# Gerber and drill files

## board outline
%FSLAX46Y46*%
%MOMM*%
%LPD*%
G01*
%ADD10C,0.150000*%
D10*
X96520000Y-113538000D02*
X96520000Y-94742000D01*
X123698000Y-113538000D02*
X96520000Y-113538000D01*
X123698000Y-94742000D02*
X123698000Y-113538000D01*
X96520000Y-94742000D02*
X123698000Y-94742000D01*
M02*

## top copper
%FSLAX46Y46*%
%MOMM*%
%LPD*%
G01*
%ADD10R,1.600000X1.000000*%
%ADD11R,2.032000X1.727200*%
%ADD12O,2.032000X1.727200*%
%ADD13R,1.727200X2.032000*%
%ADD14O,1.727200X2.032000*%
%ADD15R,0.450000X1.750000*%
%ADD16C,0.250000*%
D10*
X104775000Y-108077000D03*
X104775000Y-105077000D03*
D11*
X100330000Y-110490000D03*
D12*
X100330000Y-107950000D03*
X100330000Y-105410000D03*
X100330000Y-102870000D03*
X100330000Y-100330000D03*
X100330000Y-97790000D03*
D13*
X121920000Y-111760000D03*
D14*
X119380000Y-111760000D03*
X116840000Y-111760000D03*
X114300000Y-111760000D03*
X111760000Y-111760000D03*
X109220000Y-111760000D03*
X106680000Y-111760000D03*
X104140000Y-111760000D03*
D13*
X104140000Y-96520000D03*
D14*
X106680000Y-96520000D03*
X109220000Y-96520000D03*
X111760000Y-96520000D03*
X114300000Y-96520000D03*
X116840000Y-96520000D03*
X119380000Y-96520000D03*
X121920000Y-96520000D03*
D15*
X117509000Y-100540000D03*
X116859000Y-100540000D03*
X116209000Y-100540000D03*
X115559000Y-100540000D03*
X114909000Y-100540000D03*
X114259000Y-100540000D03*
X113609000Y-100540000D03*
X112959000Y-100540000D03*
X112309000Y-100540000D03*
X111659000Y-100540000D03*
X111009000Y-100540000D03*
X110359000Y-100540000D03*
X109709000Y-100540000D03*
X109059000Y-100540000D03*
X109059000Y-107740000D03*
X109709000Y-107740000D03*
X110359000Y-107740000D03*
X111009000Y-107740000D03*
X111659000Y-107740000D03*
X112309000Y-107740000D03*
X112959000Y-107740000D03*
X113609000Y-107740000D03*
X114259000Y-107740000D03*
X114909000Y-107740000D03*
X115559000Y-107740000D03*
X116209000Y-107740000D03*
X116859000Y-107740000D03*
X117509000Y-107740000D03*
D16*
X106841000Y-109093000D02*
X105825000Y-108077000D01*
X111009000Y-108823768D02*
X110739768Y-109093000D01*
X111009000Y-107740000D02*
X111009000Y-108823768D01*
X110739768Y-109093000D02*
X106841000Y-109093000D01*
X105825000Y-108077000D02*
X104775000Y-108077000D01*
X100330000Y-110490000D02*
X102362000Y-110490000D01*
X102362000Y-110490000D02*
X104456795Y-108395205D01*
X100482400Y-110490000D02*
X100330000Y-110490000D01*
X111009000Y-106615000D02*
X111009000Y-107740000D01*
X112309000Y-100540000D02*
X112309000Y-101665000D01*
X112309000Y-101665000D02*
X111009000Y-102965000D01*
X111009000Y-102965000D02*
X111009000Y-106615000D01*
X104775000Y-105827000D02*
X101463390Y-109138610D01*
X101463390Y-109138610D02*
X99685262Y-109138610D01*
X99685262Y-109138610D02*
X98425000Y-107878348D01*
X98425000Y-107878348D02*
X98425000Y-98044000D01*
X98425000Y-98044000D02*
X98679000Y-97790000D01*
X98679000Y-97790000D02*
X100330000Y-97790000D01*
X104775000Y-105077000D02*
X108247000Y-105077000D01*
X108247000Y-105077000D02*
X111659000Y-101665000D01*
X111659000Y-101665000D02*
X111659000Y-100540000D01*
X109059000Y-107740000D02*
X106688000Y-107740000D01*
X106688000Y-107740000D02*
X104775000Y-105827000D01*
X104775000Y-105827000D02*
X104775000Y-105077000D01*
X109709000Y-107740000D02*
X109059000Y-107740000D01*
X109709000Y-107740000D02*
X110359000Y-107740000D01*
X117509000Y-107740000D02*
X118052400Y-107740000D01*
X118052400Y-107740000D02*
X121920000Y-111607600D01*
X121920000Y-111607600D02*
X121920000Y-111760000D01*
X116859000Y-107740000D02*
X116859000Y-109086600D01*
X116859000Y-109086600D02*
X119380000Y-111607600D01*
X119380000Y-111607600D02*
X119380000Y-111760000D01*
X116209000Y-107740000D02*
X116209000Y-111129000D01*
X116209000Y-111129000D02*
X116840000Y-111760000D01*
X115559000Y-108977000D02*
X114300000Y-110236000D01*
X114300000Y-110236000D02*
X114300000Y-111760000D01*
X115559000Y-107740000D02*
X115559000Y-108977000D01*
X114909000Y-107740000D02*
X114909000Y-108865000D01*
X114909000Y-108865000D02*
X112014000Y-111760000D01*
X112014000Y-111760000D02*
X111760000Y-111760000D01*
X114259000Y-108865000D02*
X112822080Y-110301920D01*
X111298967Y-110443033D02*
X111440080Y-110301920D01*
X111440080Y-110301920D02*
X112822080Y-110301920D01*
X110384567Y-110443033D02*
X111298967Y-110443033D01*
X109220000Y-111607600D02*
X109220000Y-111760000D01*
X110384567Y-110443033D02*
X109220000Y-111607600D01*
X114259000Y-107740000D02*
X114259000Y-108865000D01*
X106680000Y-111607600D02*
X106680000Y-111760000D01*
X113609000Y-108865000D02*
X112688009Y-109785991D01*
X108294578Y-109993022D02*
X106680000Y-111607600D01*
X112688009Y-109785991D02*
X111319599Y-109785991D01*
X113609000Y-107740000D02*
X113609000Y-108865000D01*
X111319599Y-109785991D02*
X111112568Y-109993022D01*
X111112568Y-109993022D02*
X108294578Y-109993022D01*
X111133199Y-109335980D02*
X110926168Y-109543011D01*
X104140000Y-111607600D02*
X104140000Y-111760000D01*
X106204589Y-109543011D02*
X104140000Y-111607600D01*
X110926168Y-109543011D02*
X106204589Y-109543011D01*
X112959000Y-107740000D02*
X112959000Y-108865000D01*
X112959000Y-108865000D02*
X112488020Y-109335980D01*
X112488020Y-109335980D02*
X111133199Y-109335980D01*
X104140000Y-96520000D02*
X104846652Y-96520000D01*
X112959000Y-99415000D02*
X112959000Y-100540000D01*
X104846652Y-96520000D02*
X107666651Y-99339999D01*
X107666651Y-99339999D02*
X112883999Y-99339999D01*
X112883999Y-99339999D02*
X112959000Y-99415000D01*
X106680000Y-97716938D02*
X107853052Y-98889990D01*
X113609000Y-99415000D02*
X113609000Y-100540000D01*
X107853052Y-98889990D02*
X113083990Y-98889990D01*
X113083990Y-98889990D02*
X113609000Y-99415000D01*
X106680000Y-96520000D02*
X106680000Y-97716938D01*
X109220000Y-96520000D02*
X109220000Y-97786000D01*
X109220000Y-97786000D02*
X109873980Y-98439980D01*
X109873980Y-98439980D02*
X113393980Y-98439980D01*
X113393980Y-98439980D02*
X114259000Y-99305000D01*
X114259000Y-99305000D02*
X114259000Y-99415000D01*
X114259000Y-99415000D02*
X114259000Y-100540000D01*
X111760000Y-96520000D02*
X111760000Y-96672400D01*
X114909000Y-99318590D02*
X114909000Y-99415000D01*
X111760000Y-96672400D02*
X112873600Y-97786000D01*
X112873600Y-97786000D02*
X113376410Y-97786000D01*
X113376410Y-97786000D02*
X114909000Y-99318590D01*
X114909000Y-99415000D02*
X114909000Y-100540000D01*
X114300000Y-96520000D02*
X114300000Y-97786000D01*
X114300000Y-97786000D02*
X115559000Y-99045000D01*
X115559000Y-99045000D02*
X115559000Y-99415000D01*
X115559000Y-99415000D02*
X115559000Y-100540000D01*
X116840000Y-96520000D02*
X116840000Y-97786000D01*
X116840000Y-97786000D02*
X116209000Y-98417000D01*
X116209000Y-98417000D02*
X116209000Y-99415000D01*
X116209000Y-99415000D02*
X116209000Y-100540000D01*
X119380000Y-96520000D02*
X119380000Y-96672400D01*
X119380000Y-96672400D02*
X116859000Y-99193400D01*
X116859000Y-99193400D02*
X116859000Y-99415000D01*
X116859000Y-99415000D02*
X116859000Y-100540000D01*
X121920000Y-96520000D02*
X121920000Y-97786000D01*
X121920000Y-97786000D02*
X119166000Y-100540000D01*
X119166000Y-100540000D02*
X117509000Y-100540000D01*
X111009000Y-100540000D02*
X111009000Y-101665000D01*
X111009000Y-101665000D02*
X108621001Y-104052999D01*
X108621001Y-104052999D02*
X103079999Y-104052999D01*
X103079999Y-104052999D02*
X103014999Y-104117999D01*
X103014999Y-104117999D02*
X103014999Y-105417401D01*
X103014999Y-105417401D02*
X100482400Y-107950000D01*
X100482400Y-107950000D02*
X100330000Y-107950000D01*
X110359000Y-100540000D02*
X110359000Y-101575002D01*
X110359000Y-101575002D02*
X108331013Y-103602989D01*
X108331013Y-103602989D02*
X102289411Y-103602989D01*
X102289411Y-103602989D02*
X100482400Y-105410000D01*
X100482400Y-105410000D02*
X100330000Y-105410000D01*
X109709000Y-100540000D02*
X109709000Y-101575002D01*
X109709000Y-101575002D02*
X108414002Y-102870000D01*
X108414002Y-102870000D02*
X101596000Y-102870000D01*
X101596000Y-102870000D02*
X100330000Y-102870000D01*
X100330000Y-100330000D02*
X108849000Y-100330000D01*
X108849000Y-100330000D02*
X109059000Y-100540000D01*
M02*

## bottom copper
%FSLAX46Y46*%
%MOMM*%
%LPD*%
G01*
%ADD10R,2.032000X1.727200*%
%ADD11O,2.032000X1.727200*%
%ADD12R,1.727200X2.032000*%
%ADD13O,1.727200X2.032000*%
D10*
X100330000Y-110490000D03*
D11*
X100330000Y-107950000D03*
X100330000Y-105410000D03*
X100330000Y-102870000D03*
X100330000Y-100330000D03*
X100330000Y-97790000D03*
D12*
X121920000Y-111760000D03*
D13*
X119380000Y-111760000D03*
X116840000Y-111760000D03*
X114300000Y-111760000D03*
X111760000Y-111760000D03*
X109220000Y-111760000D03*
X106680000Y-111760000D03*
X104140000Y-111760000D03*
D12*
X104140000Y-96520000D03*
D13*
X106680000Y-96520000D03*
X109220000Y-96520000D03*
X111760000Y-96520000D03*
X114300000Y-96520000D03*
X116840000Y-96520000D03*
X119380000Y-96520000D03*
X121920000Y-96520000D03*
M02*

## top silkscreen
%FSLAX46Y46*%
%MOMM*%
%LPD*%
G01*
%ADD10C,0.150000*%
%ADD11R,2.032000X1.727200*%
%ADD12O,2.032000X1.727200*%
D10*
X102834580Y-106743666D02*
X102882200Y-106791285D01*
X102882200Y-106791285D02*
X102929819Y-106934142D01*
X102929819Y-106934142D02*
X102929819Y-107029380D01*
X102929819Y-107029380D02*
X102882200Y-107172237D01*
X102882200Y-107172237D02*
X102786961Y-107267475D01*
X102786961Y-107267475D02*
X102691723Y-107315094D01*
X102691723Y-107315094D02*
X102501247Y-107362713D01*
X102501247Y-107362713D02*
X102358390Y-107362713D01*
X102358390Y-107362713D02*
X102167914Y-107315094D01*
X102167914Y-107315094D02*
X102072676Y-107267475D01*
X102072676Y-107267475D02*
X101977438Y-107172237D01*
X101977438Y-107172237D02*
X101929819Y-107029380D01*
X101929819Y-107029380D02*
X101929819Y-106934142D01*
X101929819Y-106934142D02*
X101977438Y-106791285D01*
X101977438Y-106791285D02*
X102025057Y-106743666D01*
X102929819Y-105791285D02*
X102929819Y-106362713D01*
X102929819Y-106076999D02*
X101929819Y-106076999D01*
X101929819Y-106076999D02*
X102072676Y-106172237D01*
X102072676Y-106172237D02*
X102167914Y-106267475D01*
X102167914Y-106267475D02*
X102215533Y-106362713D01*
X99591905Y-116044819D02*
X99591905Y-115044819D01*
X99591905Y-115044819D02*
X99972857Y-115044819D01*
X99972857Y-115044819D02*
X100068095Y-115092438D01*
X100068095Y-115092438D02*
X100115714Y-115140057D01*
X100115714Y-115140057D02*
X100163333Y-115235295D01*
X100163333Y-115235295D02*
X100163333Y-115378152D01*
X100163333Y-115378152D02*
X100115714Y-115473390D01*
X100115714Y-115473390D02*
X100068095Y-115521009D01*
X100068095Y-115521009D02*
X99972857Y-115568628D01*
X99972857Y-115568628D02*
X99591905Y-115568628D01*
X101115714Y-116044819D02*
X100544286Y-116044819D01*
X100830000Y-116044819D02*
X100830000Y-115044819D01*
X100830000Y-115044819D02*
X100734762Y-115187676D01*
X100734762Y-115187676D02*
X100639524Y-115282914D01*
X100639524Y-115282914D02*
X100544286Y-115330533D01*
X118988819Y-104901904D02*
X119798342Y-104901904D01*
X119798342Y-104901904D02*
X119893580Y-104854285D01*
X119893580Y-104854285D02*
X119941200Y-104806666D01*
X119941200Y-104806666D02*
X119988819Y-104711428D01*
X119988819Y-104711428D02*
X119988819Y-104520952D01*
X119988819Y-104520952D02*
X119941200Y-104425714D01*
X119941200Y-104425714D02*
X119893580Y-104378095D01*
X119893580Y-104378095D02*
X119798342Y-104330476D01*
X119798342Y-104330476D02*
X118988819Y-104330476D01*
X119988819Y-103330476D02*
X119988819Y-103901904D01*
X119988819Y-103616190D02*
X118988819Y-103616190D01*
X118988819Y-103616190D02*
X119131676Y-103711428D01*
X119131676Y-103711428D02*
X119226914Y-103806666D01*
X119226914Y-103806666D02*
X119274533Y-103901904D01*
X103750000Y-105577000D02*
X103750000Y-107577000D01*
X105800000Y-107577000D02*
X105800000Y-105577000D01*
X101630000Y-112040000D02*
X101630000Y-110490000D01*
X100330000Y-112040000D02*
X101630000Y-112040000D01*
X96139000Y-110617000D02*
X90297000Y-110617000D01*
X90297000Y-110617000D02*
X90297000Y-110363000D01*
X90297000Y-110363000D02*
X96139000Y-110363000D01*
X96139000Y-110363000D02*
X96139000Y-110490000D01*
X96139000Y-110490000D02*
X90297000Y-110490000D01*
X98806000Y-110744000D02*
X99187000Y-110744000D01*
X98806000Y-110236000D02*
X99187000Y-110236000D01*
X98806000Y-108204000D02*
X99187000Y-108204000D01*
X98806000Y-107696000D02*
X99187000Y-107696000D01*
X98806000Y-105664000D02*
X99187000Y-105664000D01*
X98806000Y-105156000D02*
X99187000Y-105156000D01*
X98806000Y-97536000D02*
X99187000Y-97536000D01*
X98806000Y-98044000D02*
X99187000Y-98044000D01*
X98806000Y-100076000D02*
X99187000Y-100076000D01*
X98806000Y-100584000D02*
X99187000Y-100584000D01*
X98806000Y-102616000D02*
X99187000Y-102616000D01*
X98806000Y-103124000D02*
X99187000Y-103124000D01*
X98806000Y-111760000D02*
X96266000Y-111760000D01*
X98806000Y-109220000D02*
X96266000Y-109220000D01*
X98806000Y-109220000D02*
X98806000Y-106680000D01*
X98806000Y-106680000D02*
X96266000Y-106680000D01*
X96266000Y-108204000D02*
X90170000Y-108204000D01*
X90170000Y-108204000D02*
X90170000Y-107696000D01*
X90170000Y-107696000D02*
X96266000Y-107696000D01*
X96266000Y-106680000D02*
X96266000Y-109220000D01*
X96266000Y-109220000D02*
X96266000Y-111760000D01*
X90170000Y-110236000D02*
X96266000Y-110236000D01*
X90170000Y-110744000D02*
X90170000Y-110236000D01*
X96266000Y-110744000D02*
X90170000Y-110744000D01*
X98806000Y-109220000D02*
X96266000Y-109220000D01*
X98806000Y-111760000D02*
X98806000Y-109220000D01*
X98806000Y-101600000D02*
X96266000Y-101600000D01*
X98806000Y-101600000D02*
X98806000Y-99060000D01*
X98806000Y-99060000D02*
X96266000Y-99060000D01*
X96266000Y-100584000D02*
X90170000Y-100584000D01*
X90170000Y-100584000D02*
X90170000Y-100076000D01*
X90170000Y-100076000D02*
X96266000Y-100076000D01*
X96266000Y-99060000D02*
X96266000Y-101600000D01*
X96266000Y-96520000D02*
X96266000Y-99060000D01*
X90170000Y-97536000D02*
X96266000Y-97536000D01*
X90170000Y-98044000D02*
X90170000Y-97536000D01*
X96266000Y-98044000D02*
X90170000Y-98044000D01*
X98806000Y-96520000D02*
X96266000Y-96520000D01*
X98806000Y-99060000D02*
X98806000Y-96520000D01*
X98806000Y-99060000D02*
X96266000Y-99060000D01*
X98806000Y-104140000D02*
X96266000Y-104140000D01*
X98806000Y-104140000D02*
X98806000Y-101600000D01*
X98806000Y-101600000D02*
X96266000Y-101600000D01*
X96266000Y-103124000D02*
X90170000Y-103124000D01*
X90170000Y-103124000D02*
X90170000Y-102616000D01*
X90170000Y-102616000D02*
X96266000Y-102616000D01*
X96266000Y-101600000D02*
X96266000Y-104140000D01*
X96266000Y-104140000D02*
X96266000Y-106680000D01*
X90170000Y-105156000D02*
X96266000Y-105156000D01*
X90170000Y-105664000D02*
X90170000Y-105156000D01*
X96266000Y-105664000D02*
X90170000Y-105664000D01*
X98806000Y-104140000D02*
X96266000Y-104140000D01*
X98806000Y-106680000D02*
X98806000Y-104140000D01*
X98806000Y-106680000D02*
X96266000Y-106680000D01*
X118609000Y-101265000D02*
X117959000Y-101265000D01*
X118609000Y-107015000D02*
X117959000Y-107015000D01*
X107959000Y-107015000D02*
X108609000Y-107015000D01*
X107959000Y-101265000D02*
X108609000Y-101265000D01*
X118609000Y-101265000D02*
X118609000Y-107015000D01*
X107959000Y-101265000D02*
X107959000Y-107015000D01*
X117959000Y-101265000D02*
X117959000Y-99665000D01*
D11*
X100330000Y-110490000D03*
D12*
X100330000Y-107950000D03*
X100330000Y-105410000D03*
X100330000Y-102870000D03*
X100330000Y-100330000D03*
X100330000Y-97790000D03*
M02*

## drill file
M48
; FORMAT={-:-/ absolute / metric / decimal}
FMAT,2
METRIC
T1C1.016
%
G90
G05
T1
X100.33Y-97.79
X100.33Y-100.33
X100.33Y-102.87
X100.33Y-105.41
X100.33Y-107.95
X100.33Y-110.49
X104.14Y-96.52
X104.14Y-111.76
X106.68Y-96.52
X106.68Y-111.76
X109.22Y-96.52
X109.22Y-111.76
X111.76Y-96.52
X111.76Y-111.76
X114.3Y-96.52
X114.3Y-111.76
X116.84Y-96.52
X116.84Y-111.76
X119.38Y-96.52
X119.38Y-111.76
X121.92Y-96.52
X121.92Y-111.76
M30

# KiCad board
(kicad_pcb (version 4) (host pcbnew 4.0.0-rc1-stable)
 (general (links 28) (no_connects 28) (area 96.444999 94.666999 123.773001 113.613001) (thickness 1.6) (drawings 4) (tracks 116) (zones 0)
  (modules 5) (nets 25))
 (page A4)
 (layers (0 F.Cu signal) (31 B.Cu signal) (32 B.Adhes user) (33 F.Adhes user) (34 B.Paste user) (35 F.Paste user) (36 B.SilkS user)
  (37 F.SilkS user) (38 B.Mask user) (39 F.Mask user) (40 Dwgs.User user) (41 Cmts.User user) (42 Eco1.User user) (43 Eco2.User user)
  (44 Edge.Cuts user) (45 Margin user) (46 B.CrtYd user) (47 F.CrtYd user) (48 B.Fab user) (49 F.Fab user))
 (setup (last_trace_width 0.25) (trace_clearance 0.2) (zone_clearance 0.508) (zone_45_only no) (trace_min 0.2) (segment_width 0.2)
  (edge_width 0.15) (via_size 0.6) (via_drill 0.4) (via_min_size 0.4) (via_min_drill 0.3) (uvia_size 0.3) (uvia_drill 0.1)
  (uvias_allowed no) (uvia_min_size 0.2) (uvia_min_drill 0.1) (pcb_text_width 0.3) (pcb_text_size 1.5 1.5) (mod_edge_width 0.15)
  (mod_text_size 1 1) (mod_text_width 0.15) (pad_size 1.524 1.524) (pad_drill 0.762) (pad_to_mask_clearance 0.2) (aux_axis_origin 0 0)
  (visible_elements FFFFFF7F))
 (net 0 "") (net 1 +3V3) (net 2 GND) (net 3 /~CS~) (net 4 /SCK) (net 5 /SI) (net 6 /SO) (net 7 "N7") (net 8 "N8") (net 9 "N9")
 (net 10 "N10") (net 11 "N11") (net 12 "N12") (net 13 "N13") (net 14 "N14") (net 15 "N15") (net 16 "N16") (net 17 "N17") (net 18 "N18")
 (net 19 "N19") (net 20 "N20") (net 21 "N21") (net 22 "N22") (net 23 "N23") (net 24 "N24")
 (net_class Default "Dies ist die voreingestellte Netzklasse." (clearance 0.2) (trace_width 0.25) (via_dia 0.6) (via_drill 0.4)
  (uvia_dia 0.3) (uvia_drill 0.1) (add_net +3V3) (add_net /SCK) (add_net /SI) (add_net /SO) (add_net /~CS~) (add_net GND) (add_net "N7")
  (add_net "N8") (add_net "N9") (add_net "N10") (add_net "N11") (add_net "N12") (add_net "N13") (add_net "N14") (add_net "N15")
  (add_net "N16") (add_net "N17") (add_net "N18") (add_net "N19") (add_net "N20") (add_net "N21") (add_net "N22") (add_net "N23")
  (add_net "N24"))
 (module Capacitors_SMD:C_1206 (layer F.Cu) (at 104.775 106.577 90)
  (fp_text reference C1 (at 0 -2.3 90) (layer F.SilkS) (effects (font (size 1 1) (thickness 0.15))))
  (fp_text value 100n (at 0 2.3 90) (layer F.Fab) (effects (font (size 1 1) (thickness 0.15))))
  (fp_line (start 1 -1.025) (end -1 -1.025) (layer F.SilkS) (width 0.15))
  (fp_line (start -1 1.025) (end 1 1.025) (layer F.SilkS) (width 0.15))
  (pad 1 smd rect (at -1.5 0 90) (size 1 1.6) (layers F.Cu F.Paste F.Mask) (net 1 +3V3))
  (pad 2 smd rect (at 1.5 0 90) (size 1 1.6) (layers F.Cu F.Paste F.Mask) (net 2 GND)))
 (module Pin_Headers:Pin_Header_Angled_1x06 (layer F.Cu) (at 100.33 110.49 180)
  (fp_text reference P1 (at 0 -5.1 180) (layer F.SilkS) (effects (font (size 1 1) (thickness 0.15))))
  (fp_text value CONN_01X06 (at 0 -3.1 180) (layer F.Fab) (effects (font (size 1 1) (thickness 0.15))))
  (fp_line (start -1.3 -1.55) (end -1.3 0) (layer F.SilkS) (width 0.15))
  (fp_line (start 0 -1.55) (end -1.3 -1.55) (layer F.SilkS) (width 0.15))
  (fp_line (start 4.191 -0.127) (end 10.033 -0.127) (layer F.SilkS) (width 0.15))
  (fp_line (start 10.033 -0.127) (end 10.033 0.127) (layer F.SilkS) (width 0.15))
  (fp_line (start 10.033 0.127) (end 4.191 0.127) (layer F.SilkS) (width 0.15))
  (fp_line (start 4.191 0.127) (end 4.191 0) (layer F.SilkS) (width 0.15))
  (fp_line (start 4.191 0) (end 10.033 0) (layer F.SilkS) (width 0.15))
  (fp_line (start 1.524 -0.254) (end 1.143 -0.254) (layer F.SilkS) (width 0.15))
  (fp_line (start 1.524 0.254) (end 1.143 0.254) (layer F.SilkS) (width 0.15))
  (fp_line (start 1.524 2.286) (end 1.143 2.286) (layer F.SilkS) (width 0.15))
  (fp_line (start 1.524 2.794) (end 1.143 2.794) (layer F.SilkS) (width 0.15))
  (fp_line (start 1.524 4.826) (end 1.143 4.826) (layer F.SilkS) (width 0.15))
  (fp_line (start 1.524 5.334) (end 1.143 5.334) (layer F.SilkS) (width 0.15))
  (fp_line (start 1.524 12.954) (end 1.143 12.954) (layer F.SilkS) (width 0.15))
  (fp_line (start 1.524 12.446) (end 1.143 12.446) (layer F.SilkS) (width 0.15))
  (fp_line (start 1.524 10.414) (end 1.143 10.414) (layer F.SilkS) (width 0.15))
  (fp_line (start 1.524 9.906) (end 1.143 9.906) (layer F.SilkS) (width 0.15))
  (fp_line (start 1.524 7.874) (end 1.143 7.874) (layer F.SilkS) (width 0.15))
  (fp_line (start 1.524 7.366) (end 1.143 7.366) (layer F.SilkS) (width 0.15))
  (fp_line (start 1.524 -1.27) (end 4.064 -1.27) (layer F.SilkS) (width 0.15))
  (fp_line (start 1.524 1.27) (end 4.064 1.27) (layer F.SilkS) (width 0.15))
  (fp_line (start 1.524 1.27) (end 1.524 3.81) (layer F.SilkS) (width 0.15))
  (fp_line (start 1.524 3.81) (end 4.064 3.81) (layer F.SilkS) (width 0.15))
  (fp_line (start 4.064 2.286) (end 10.16 2.286) (layer F.SilkS) (width 0.15))
  (fp_line (start 10.16 2.286) (end 10.16 2.794) (layer F.SilkS) (width 0.15))
  (fp_line (start 10.16 2.794) (end 4.064 2.794) (layer F.SilkS) (width 0.15))
  (fp_line (start 4.064 3.81) (end 4.064 1.27) (layer F.SilkS) (width 0.15))
  (fp_line (start 4.064 1.27) (end 4.064 -1.27) (layer F.SilkS) (width 0.15))
  (fp_line (start 10.16 0.254) (end 4.064 0.254) (layer F.SilkS) (width 0.15))
  (fp_line (start 10.16 -0.254) (end 10.16 0.254) (layer F.SilkS) (width 0.15))
  (fp_line (start 4.064 -0.254) (end 10.16 -0.254) (layer F.SilkS) (width 0.15))
  (fp_line (start 1.524 1.27) (end 4.064 1.27) (layer F.SilkS) (width 0.15))
  (fp_line (start 1.524 -1.27) (end 1.524 1.27) (layer F.SilkS) (width 0.15))
  (fp_line (start 1.524 8.89) (end 4.064 8.89) (layer F.SilkS) (width 0.15))
  (fp_line (start 1.524 8.89) (end 1.524 11.43) (layer F.SilkS) (width 0.15))
  (fp_line (start 1.524 11.43) (end 4.064 11.43) (layer F.SilkS) (width 0.15))
  (fp_line (start 4.064 9.906) (end 10.16 9.906) (layer F.SilkS) (width 0.15))
  (fp_line (start 10.16 9.906) (end 10.16 10.414) (layer F.SilkS) (width 0.15))
  (fp_line (start 10.16 10.414) (end 4.064 10.414) (layer F.SilkS) (width 0.15))
  (fp_line (start 4.064 11.43) (end 4.064 8.89) (layer F.SilkS) (width 0.15))
  (fp_line (start 4.064 13.97) (end 4.064 11.43) (layer F.SilkS) (width 0.15))
  (fp_line (start 10.16 12.954) (end 4.064 12.954) (layer F.SilkS) (width 0.15))
  (fp_line (start 10.16 12.446) (end 10.16 12.954) (layer F.SilkS) (width 0.15))
  (fp_line (start 4.064 12.446) (end 10.16 12.446) (layer F.SilkS) (width 0.15))
  (fp_line (start 1.524 13.97) (end 4.064 13.97) (layer F.SilkS) (width 0.15))
  (fp_line (start 1.524 11.43) (end 1.524 13.97) (layer F.SilkS) (width 0.15))
  (fp_line (start 1.524 11.43) (end 4.064 11.43) (layer F.SilkS) (width 0.15))
  (fp_line (start 1.524 6.35) (end 4.064 6.35) (layer F.SilkS) (width 0.15))
  (fp_line (start 1.524 6.35) (end 1.524 8.89) (layer F.SilkS) (width 0.15))
  (fp_line (start 1.524 8.89) (end 4.064 8.89) (layer F.SilkS) (width 0.15))
  (fp_line (start 4.064 7.366) (end 10.16 7.366) (layer F.SilkS) (width 0.15))
  (fp_line (start 10.16 7.366) (end 10.16 7.874) (layer F.SilkS) (width 0.15))
  (fp_line (start 10.16 7.874) (end 4.064 7.874) (layer F.SilkS) (width 0.15))
  (fp_line (start 4.064 8.89) (end 4.064 6.35) (layer F.SilkS) (width 0.15))
  (fp_line (start 4.064 6.35) (end 4.064 3.81) (layer F.SilkS) (width 0.15))
  (fp_line (start 10.16 5.334) (end 4.064 5.334) (layer F.SilkS) (width 0.15))
  (fp_line (start 10.16 4.826) (end 10.16 5.334) (layer F.SilkS) (width 0.15))
  (fp_line (start 4.064 4.826) (end 10.16 4.826) (layer F.SilkS) (width 0.15))
  (fp_line (start 1.524 6.35) (end 4.064 6.35) (layer F.SilkS) (width 0.15))
  (fp_line (start 1.524 3.81) (end 1.524 6.35) (layer F.SilkS) (width 0.15))
  (fp_line (start 1.524 3.81) (end 4.064 3.81) (layer F.SilkS) (width 0.15))
  (pad 1 thru_hole rect (at 0 0 180) (size 2.032 1.7272) (drill 1.016) (layers *.Cu *.Mask F.SilkS) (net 1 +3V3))
  (pad 2 thru_hole oval (at 0 2.54 180) (size 2.032 1.7272) (drill 1.016) (layers *.Cu *.Mask F.SilkS) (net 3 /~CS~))
  (pad 3 thru_hole oval (at 0 5.08 180) (size 2.032 1.7272) (drill 1.016) (layers *.Cu *.Mask F.SilkS) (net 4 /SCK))
  (pad 4 thru_hole oval (at 0 7.62 180) (size 2.032 1.7272) (drill 1.016) (layers *.Cu *.Mask F.SilkS) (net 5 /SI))
  (pad 5 thru_hole oval (at 0 10.16 180) (size 2.032 1.7272) (drill 1.016) (layers *.Cu *.Mask F.SilkS) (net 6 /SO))
  (pad 6 thru_hole oval (at 0 12.7 180) (size 2.032 1.7272) (drill 1.016) (layers *.Cu *.Mask F.SilkS) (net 2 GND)))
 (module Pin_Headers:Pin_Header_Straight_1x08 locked (layer B.Cu) (at 121.92 111.76 90)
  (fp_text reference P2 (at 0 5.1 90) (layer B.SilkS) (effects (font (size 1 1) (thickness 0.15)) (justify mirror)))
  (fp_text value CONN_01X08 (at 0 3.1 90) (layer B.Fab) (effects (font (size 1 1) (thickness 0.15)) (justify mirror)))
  (pad 1 thru_hole rect (at 0 0 90) (size 2.032 1.7272) (drill 1.016) (layers *.Cu *.Mask B.SilkS) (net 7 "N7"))
  (pad 2 thru_hole oval (at 0 -2.54 90) (size 2.032 1.7272) (drill 1.016) (layers *.Cu *.Mask B.SilkS) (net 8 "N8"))
  (pad 3 thru_hole oval (at 0 -5.08 90) (size 2.032 1.7272) (drill 1.016) (layers *.Cu *.Mask B.SilkS) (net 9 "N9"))
  (pad 4 thru_hole oval (at 0 -7.62 90) (size 2.032 1.7272) (drill 1.016) (layers *.Cu *.Mask B.SilkS) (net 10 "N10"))
  (pad 5 thru_hole oval (at 0 -10.16 90) (size 2.032 1.7272) (drill 1.016) (layers *.Cu *.Mask B.SilkS) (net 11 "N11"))
  (pad 6 thru_hole oval (at 0 -12.7 90) (size 2.032 1.7272) (drill 1.016) (layers *.Cu *.Mask B.SilkS) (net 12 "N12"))
  (pad 7 thru_hole oval (at 0 -15.24 90) (size 2.032 1.7272) (drill 1.016) (layers *.Cu *.Mask B.SilkS) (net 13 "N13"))
  (pad 8 thru_hole oval (at 0 -17.78 90) (size 2.032 1.7272) (drill 1.016) (layers *.Cu *.Mask B.SilkS) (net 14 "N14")))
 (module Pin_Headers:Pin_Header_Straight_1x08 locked (layer B.Cu) (at 104.14 96.52 270)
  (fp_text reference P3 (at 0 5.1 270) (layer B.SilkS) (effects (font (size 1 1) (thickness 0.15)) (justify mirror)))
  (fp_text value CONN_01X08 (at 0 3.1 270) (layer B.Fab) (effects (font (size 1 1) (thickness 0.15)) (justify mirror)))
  (pad 1 thru_hole rect (at 0 0 270) (size 2.032 1.7272) (drill 1.016) (layers *.Cu *.Mask B.SilkS) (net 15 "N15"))
  (pad 2 thru_hole oval (at 0 -2.54 270) (size 2.032 1.7272) (drill 1.016) (layers *.Cu *.Mask B.SilkS) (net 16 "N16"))
  (pad 3 thru_hole oval (at 0 -5.08 270) (size 2.032 1.7272) (drill 1.016) (layers *.Cu *.Mask B.SilkS) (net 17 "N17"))
  (pad 4 thru_hole oval (at 0 -7.62 270) (size 2.032 1.7272) (drill 1.016) (layers *.Cu *.Mask B.SilkS) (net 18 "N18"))
  (pad 5 thru_hole oval (at 0 -10.16 270) (size 2.032 1.7272) (drill 1.016) (layers *.Cu *.Mask B.SilkS) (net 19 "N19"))
  (pad 6 thru_hole oval (at 0 -12.7 270) (size 2.032 1.7272) (drill 1.016) (layers *.Cu *.Mask B.SilkS) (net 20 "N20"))
  (pad 7 thru_hole oval (at 0 -15.24 270) (size 2.032 1.7272) (drill 1.016) (layers *.Cu *.Mask B.SilkS) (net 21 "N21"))
  (pad 8 thru_hole oval (at 0 -17.78 270) (size 2.032 1.7272) (drill 1.016) (layers *.Cu *.Mask B.SilkS) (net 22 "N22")))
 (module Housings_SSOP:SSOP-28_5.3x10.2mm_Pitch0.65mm (layer F.Cu) (at 113.284 104.14 270)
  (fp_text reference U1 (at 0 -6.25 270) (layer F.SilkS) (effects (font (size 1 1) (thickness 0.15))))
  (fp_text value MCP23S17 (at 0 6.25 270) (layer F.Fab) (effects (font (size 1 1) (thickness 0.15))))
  (fp_line (start -2.875 -5.325) (end -2.875 -4.675) (layer F.SilkS) (width 0.15))
  (fp_line (start 2.875 -5.325) (end 2.875 -4.675) (layer F.SilkS) (width 0.15))
  (fp_line (start 2.875 5.325) (end 2.875 4.675) (layer F.SilkS) (width 0.15))
  (fp_line (start -2.875 5.325) (end -2.875 4.675) (layer F.SilkS) (width 0.15))
  (fp_line (start -2.875 -5.325) (end 2.875 -5.325) (layer F.SilkS) (width 0.15))
  (fp_line (start -2.875 5.325) (end 2.875 5.325) (layer F.SilkS) (width 0.15))
  (fp_line (start -2.875 -4.675) (end -4.475 -4.675) (layer F.SilkS) (width 0.15))
  (pad 1 smd rect (at -3.6 -4.225 270) (size 1.75 0.45) (layers F.Cu F.Paste F.Mask) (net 22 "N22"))
  (pad 2 smd rect (at -3.6 -3.575 270) (size 1.75 0.45) (layers F.Cu F.Paste F.Mask) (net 21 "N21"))
  (pad 3 smd rect (at -3.6 -2.925 270) (size 1.75 0.45) (layers F.Cu F.Paste F.Mask) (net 20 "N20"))
  (pad 4 smd rect (at -3.6 -2.275 270) (size 1.75 0.45) (layers F.Cu F.Paste F.Mask) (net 19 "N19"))
  (pad 5 smd rect (at -3.6 -1.625 270) (size 1.75 0.45) (layers F.Cu F.Paste F.Mask) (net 18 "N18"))
  (pad 6 smd rect (at -3.6 -0.975 270) (size 1.75 0.45) (layers F.Cu F.Paste F.Mask) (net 17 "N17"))
  (pad 7 smd rect (at -3.6 -0.325 270) (size 1.75 0.45) (layers F.Cu F.Paste F.Mask) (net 16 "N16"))
  (pad 8 smd rect (at -3.6 0.325 270) (size 1.75 0.45) (layers F.Cu F.Paste F.Mask) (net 15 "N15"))
  (pad 9 smd rect (at -3.6 0.975 270) (size 1.75 0.45) (layers F.Cu F.Paste F.Mask) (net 1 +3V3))
  (pad 10 smd rect (at -3.6 1.625 270) (size 1.75 0.45) (layers F.Cu F.Paste F.Mask) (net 2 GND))
  (pad 11 smd rect (at -3.6 2.275 270) (size 1.75 0.45) (layers F.Cu F.Paste F.Mask) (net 3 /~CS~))
  (pad 12 smd rect (at -3.6 2.925 270) (size 1.75 0.45) (layers F.Cu F.Paste F.Mask) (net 4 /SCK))
  (pad 13 smd rect (at -3.6 3.575 270) (size 1.75 0.45) (layers F.Cu F.Paste F.Mask) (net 5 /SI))
  (pad 14 smd rect (at -3.6 4.225 270) (size 1.75 0.45) (layers F.Cu F.Paste F.Mask) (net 6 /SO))
  (pad 15 smd rect (at 3.6 4.225 270) (size 1.75 0.45) (layers F.Cu F.Paste F.Mask) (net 2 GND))
  (pad 16 smd rect (at 3.6 3.575 270) (size 1.75 0.45) (layers F.Cu F.Paste F.Mask) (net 2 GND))
  (pad 17 smd rect (at 3.6 2.925 270) (size 1.75 0.45) (layers F.Cu F.Paste F.Mask) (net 2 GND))
  (pad 18 smd rect (at 3.6 2.275 270) (size 1.75 0.45) (layers F.Cu F.Paste F.Mask) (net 1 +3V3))
  (pad 19 smd rect (at 3.6 1.625 270) (size 1.75 0.45) (layers F.Cu F.Paste F.Mask) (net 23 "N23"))
  (pad 20 smd rect (at 3.6 0.975 270) (size 1.75 0.45) (layers F.Cu F.Paste F.Mask) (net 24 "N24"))
  (pad 21 smd rect (at 3.6 0.325 270) (size 1.75 0.45) (layers F.Cu F.Paste F.Mask) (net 14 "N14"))
  (pad 22 smd rect (at 3.6 -0.325 270) (size 1.75 0.45) (layers F.Cu F.Paste F.Mask) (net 13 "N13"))
  (pad 23 smd rect (at 3.6 -0.975 270) (size 1.75 0.45) (layers F.Cu F.Paste F.Mask) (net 12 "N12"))
  (pad 24 smd rect (at 3.6 -1.625 270) (size 1.75 0.45) (layers F.Cu F.Paste F.Mask) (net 11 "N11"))
  (pad 25 smd rect (at 3.6 -2.275 270) (size 1.75 0.45) (layers F.Cu F.Paste F.Mask) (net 10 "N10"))
  (pad 26 smd rect (at 3.6 -2.925 270) (size 1.75 0.45) (layers F.Cu F.Paste F.Mask) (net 9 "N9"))
  (pad 27 smd rect (at 3.6 -3.575 270) (size 1.75 0.45) (layers F.Cu F.Paste F.Mask) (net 8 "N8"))
  (pad 28 smd rect (at 3.6 -4.225 270) (size 1.75 0.45) (layers F.Cu F.Paste F.Mask) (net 7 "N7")))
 (gr_line (start 96.52 113.538) (end 96.52 94.742) (layer Edge.Cuts) (width 0.15))
 (gr_line (start 123.698 113.538) (end 96.52 113.538) (layer Edge.Cuts) (width 0.15))
 (gr_line (start 123.698 94.742) (end 123.698 113.538) (layer Edge.Cuts) (width 0.15))
 (gr_line (start 96.52 94.742) (end 123.698 94.742) (layer Edge.Cuts) (width 0.15))
 (segment (start 106.841 109.093) (end 105.825 108.077) (width 0.25) (layer F.Cu) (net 1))
 (segment (start 111.009 108.823768) (end 110.739768 109.093) (width 0.25) (layer F.Cu) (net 1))
 (segment (start 111.009 107.74) (end 111.009 108.823768) (width 0.25) (layer F.Cu) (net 1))
 (segment (start 110.739768 109.093) (end 106.841 109.093) (width 0.25) (layer F.Cu) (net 1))
 (segment (start 105.825 108.077) (end 104.775 108.077) (width 0.25) (layer F.Cu) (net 1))
 (segment (start 100.33 110.49) (end 102.362 110.49) (width 0.25) (layer F.Cu) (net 1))
 (segment (start 102.362 110.49) (end 104.456795 108.395205) (width 0.25) (layer F.Cu) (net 1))
 (segment (start 100.4824 110.49) (end 100.33 110.49) (width 0.25) (layer F.Cu) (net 1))
 (segment (start 111.009 106.615) (end 111.009 107.74) (width 0.25) (layer F.Cu) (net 1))
 (segment (start 112.309 100.54) (end 112.309 101.665) (width 0.25) (layer F.Cu) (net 1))
 (segment (start 112.309 101.665) (end 111.009 102.965) (width 0.25) (layer F.Cu) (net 1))
 (segment (start 111.009 102.965) (end 111.009 106.615) (width 0.25) (layer F.Cu) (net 1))
 (segment (start 104.775 105.827) (end 101.46339 109.13861) (width 0.25) (layer F.Cu) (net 2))
 (segment (start 101.46339 109.13861) (end 99.685262 109.13861) (width 0.25) (layer F.Cu) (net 2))
 (segment (start 99.685262 109.13861) (end 98.425 107.878348) (width 0.25) (layer F.Cu) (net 2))
 (segment (start 98.425 107.878348) (end 98.425 98.044) (width 0.25) (layer F.Cu) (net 2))
 (segment (start 98.425 98.044) (end 98.679 97.79) (width 0.25) (layer F.Cu) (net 2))
 (segment (start 98.679 97.79) (end 100.33 97.79) (width 0.25) (layer F.Cu) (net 2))
 (segment (start 104.775 105.077) (end 108.247 105.077) (width 0.25) (layer F.Cu) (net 2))
 (segment (start 108.247 105.077) (end 111.659 101.665) (width 0.25) (layer F.Cu) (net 2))
 (segment (start 111.659 101.665) (end 111.659 100.54) (width 0.25) (layer F.Cu) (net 2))
 (segment (start 109.059 107.74) (end 106.688 107.74) (width 0.25) (layer F.Cu) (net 2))
 (segment (start 106.688 107.74) (end 104.775 105.827) (width 0.25) (layer F.Cu) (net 2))
 (segment (start 104.775 105.827) (end 104.775 105.077) (width 0.25) (layer F.Cu) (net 2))
 (segment (start 109.709 107.74) (end 109.059 107.74) (width 0.25) (layer F.Cu) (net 2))
 (segment (start 109.709 107.74) (end 110.359 107.74) (width 0.25) (layer F.Cu) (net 2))
 (segment (start 117.509 107.74) (end 118.0524 107.74) (width 0.25) (layer F.Cu) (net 7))
 (segment (start 118.0524 107.74) (end 121.92 111.6076) (width 0.25) (layer F.Cu) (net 7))
 (segment (start 121.92 111.6076) (end 121.92 111.76) (width 0.25) (layer F.Cu) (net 7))
 (segment (start 116.859 107.74) (end 116.859 109.0866) (width 0.25) (layer F.Cu) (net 8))
 (segment (start 116.859 109.0866) (end 119.38 111.6076) (width 0.25) (layer F.Cu) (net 8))
 (segment (start 119.38 111.6076) (end 119.38 111.76) (width 0.25) (layer F.Cu) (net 8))
 (segment (start 116.209 107.74) (end 116.209 111.129) (width 0.25) (layer F.Cu) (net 9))
 (segment (start 116.209 111.129) (end 116.84 111.76) (width 0.25) (layer F.Cu) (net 9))
 (segment (start 115.559 108.977) (end 114.3 110.236) (width 0.25) (layer F.Cu) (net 10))
 (segment (start 114.3 110.236) (end 114.3 111.76) (width 0.25) (layer F.Cu) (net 10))
 (segment (start 115.559 107.74) (end 115.559 108.977) (width 0.25) (layer F.Cu) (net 10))
 (segment (start 114.909 107.74) (end 114.909 108.865) (width 0.25) (layer F.Cu) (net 11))
 (segment (start 114.909 108.865) (end 112.014 111.76) (width 0.25) (layer F.Cu) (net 11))
 (segment (start 112.014 111.76) (end 111.76 111.76) (width 0.25) (layer F.Cu) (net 11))
 (segment (start 114.259 108.865) (end 112.82208 110.30192) (width 0.25) (layer F.Cu) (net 12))
 (segment (start 111.298967 110.443033) (end 111.44008 110.30192) (width 0.25) (layer F.Cu) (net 12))
 (segment (start 111.44008 110.30192) (end 112.82208 110.30192) (width 0.25) (layer F.Cu) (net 12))
 (segment (start 110.384567 110.443033) (end 111.298967 110.443033) (width 0.25) (layer F.Cu) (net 12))
 (segment (start 109.22 111.6076) (end 109.22 111.76) (width 0.25) (layer F.Cu) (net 12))
 (segment (start 110.384567 110.443033) (end 109.22 111.6076) (width 0.25) (layer F.Cu) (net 12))
 (segment (start 114.259 107.74) (end 114.259 108.865) (width 0.25) (layer F.Cu) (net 12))
 (segment (start 106.68 111.6076) (end 106.68 111.76) (width 0.25) (layer F.Cu) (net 13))
 (segment (start 113.609 108.865) (end 112.688009 109.785991) (width 0.25) (layer F.Cu) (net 13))
 (segment (start 108.294578 109.993022) (end 106.68 111.6076) (width 0.25) (layer F.Cu) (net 13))
 (segment (start 112.688009 109.785991) (end 111.319599 109.785991) (width 0.25) (layer F.Cu) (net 13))
 (segment (start 113.609 107.74) (end 113.609 108.865) (width 0.25) (layer F.Cu) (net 13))
 (segment (start 111.319599 109.785991) (end 111.112568 109.993022) (width 0.25) (layer F.Cu) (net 13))
 (segment (start 111.112568 109.993022) (end 108.294578 109.993022) (width 0.25) (layer F.Cu) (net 13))
 (segment (start 111.133199 109.33598) (end 110.926168 109.543011) (width 0.25) (layer F.Cu) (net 14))
 (segment (start 104.14 111.6076) (end 104.14 111.76) (width 0.25) (layer F.Cu) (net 14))
 (segment (start 106.204589 109.543011) (end 104.14 111.6076) (width 0.25) (layer F.Cu) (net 14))
 (segment (start 110.926168 109.543011) (end 106.204589 109.543011) (width 0.25) (layer F.Cu) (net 14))
 (segment (start 112.959 107.74) (end 112.959 108.865) (width 0.25) (layer F.Cu) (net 14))
 (segment (start 112.959 108.865) (end 112.48802 109.33598) (width 0.25) (layer F.Cu) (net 14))
 (segment (start 112.48802 109.33598) (end 111.133199 109.33598) (width 0.25) (layer F.Cu) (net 14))
 (segment (start 104.14 96.52) (end 104.846652 96.52) (width 0.25) (layer F.Cu) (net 15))
 (segment (start 112.959 99.415) (end 112.959 100.54) (width 0.25) (layer F.Cu) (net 15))
 (segment (start 104.846652 96.52) (end 107.666651 99.339999) (width 0.25) (layer F.Cu) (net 15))
 (segment (start 107.666651 99.339999) (end 112.883999 99.339999) (width 0.25) (layer F.Cu) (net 15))
 (segment (start 112.883999 99.339999) (end 112.959 99.415) (width 0.25) (layer F.Cu) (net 15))
 (segment (start 106.68 97.716938) (end 107.853052 98.88999) (width 0.25) (layer F.Cu) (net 16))
 (segment (start 113.609 99.415) (end 113.609 100.54) (width 0.25) (layer F.Cu) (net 16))
 (segment (start 107.853052 98.88999) (end 113.08399 98.88999) (width 0.25) (layer F.Cu) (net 16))
 (segment (start 113.08399 98.88999) (end 113.609 99.415) (width 0.25) (layer F.Cu) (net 16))
 (segment (start 106.68 96.52) (end 106.68 97.716938) (width 0.25) (layer F.Cu) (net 16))
 (segment (start 109.22 96.52) (end 109.22 97.786) (width 0.25) (layer F.Cu) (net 17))
 (segment (start 109.22 97.786) (end 109.87398 98.43998) (width 0.25) (layer F.Cu) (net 17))
 (segment (start 109.87398 98.43998) (end 113.39398 98.43998) (width 0.25) (layer F.Cu) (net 17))
 (segment (start 113.39398 98.43998) (end 114.259 99.305) (width 0.25) (layer F.Cu) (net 17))
 (segment (start 114.259 99.305) (end 114.259 99.415) (width 0.25) (layer F.Cu) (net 17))
 (segment (start 114.259 99.415) (end 114.259 100.54) (width 0.25) (layer F.Cu) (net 17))
 (segment (start 111.76 96.52) (end 111.76 96.6724) (width 0.25) (layer F.Cu) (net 18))
 (segment (start 114.909 99.31859) (end 114.909 99.415) (width 0.25) (layer F.Cu) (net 18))
 (segment (start 111.76 96.6724) (end 112.8736 97.786) (width 0.25) (layer F.Cu) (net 18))
 (segment (start 112.8736 97.786) (end 113.37641 97.786) (width 0.25) (layer F.Cu) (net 18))
 (segment (start 113.37641 97.786) (end 114.909 99.31859) (width 0.25) (layer F.Cu) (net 18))
 (segment (start 114.909 99.415) (end 114.909 100.54) (width 0.25) (layer F.Cu) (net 18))
 (segment (start 114.3 96.52) (end 114.3 97.786) (width 0.25) (layer F.Cu) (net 19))
 (segment (start 114.3 97.786) (end 115.559 99.045) (width 0.25) (layer F.Cu) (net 19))
 (segment (start 115.559 99.045) (end 115.559 99.415) (width 0.25) (layer F.Cu) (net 19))
 (segment (start 115.559 99.415) (end 115.559 100.54) (width 0.25) (layer F.Cu) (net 19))
 (segment (start 116.84 96.52) (end 116.84 97.786) (width 0.25) (layer F.Cu) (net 20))
 (segment (start 116.84 97.786) (end 116.209 98.417) (width 0.25) (layer F.Cu) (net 20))
 (segment (start 116.209 98.417) (end 116.209 99.415) (width 0.25) (layer F.Cu) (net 20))
 (segment (start 116.209 99.415) (end 116.209 100.54) (width 0.25) (layer F.Cu) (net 20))
 (segment (start 119.38 96.52) (end 119.38 96.6724) (width 0.25) (layer F.Cu) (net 21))
 (segment (start 119.38 96.6724) (end 116.859 99.1934) (width 0.25) (layer F.Cu) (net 21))
 (segment (start 116.859 99.1934) (end 116.859 99.415) (width 0.25) (layer F.Cu) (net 21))
 (segment (start 116.859 99.415) (end 116.859 100.54) (width 0.25) (layer F.Cu) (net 21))
 (segment (start 121.92 96.52) (end 121.92 97.786) (width 0.25) (layer F.Cu) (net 22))
 (segment (start 121.92 97.786) (end 119.166 100.54) (width 0.25) (layer F.Cu) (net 22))
 (segment (start 119.166 100.54) (end 117.509 100.54) (width 0.25) (layer F.Cu) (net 22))
 (segment (start 111.009 100.54) (end 111.009 101.665) (width 0.25) (layer F.Cu) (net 3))
 (segment (start 111.009 101.665) (end 108.621001 104.052999) (width 0.25) (layer F.Cu) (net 3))
 (segment (start 108.621001 104.052999) (end 103.079999 104.052999) (width 0.25) (layer F.Cu) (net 3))
 (segment (start 103.079999 104.052999) (end 103.014999 104.117999) (width 0.25) (layer F.Cu) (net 3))
 (segment (start 103.014999 104.117999) (end 103.014999 105.417401) (width 0.25) (layer F.Cu) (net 3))
 (segment (start 103.014999 105.417401) (end 100.4824 107.95) (width 0.25) (layer F.Cu) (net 3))
 (segment (start 100.4824 107.95) (end 100.33 107.95) (width 0.25) (layer F.Cu) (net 3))
 (segment (start 110.359 100.54) (end 110.359 101.575002) (width 0.25) (layer F.Cu) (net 4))
 (segment (start 110.359 101.575002) (end 108.331013 103.602989) (width 0.25) (layer F.Cu) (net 4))
 (segment (start 108.331013 103.602989) (end 102.289411 103.602989) (width 0.25) (layer F.Cu) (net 4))
 (segment (start 102.289411 103.602989) (end 100.4824 105.41) (width 0.25) (layer F.Cu) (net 4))
 (segment (start 100.4824 105.41) (end 100.33 105.41) (width 0.25) (layer F.Cu) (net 4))
 (segment (start 109.709 100.54) (end 109.709 101.575002) (width 0.25) (layer F.Cu) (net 5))
 (segment (start 109.709 101.575002) (end 108.414002 102.87) (width 0.25) (layer F.Cu) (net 5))
 (segment (start 108.414002 102.87) (end 101.596 102.87) (width 0.25) (layer F.Cu) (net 5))
 (segment (start 101.596 102.87) (end 100.33 102.87) (width 0.25) (layer F.Cu) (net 5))
 (segment (start 100.33 100.33) (end 108.849 100.33) (width 0.25) (layer F.Cu) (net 6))
 (segment (start 108.849 100.33) (end 109.059 100.54) (width 0.25) (layer F.Cu) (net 6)))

